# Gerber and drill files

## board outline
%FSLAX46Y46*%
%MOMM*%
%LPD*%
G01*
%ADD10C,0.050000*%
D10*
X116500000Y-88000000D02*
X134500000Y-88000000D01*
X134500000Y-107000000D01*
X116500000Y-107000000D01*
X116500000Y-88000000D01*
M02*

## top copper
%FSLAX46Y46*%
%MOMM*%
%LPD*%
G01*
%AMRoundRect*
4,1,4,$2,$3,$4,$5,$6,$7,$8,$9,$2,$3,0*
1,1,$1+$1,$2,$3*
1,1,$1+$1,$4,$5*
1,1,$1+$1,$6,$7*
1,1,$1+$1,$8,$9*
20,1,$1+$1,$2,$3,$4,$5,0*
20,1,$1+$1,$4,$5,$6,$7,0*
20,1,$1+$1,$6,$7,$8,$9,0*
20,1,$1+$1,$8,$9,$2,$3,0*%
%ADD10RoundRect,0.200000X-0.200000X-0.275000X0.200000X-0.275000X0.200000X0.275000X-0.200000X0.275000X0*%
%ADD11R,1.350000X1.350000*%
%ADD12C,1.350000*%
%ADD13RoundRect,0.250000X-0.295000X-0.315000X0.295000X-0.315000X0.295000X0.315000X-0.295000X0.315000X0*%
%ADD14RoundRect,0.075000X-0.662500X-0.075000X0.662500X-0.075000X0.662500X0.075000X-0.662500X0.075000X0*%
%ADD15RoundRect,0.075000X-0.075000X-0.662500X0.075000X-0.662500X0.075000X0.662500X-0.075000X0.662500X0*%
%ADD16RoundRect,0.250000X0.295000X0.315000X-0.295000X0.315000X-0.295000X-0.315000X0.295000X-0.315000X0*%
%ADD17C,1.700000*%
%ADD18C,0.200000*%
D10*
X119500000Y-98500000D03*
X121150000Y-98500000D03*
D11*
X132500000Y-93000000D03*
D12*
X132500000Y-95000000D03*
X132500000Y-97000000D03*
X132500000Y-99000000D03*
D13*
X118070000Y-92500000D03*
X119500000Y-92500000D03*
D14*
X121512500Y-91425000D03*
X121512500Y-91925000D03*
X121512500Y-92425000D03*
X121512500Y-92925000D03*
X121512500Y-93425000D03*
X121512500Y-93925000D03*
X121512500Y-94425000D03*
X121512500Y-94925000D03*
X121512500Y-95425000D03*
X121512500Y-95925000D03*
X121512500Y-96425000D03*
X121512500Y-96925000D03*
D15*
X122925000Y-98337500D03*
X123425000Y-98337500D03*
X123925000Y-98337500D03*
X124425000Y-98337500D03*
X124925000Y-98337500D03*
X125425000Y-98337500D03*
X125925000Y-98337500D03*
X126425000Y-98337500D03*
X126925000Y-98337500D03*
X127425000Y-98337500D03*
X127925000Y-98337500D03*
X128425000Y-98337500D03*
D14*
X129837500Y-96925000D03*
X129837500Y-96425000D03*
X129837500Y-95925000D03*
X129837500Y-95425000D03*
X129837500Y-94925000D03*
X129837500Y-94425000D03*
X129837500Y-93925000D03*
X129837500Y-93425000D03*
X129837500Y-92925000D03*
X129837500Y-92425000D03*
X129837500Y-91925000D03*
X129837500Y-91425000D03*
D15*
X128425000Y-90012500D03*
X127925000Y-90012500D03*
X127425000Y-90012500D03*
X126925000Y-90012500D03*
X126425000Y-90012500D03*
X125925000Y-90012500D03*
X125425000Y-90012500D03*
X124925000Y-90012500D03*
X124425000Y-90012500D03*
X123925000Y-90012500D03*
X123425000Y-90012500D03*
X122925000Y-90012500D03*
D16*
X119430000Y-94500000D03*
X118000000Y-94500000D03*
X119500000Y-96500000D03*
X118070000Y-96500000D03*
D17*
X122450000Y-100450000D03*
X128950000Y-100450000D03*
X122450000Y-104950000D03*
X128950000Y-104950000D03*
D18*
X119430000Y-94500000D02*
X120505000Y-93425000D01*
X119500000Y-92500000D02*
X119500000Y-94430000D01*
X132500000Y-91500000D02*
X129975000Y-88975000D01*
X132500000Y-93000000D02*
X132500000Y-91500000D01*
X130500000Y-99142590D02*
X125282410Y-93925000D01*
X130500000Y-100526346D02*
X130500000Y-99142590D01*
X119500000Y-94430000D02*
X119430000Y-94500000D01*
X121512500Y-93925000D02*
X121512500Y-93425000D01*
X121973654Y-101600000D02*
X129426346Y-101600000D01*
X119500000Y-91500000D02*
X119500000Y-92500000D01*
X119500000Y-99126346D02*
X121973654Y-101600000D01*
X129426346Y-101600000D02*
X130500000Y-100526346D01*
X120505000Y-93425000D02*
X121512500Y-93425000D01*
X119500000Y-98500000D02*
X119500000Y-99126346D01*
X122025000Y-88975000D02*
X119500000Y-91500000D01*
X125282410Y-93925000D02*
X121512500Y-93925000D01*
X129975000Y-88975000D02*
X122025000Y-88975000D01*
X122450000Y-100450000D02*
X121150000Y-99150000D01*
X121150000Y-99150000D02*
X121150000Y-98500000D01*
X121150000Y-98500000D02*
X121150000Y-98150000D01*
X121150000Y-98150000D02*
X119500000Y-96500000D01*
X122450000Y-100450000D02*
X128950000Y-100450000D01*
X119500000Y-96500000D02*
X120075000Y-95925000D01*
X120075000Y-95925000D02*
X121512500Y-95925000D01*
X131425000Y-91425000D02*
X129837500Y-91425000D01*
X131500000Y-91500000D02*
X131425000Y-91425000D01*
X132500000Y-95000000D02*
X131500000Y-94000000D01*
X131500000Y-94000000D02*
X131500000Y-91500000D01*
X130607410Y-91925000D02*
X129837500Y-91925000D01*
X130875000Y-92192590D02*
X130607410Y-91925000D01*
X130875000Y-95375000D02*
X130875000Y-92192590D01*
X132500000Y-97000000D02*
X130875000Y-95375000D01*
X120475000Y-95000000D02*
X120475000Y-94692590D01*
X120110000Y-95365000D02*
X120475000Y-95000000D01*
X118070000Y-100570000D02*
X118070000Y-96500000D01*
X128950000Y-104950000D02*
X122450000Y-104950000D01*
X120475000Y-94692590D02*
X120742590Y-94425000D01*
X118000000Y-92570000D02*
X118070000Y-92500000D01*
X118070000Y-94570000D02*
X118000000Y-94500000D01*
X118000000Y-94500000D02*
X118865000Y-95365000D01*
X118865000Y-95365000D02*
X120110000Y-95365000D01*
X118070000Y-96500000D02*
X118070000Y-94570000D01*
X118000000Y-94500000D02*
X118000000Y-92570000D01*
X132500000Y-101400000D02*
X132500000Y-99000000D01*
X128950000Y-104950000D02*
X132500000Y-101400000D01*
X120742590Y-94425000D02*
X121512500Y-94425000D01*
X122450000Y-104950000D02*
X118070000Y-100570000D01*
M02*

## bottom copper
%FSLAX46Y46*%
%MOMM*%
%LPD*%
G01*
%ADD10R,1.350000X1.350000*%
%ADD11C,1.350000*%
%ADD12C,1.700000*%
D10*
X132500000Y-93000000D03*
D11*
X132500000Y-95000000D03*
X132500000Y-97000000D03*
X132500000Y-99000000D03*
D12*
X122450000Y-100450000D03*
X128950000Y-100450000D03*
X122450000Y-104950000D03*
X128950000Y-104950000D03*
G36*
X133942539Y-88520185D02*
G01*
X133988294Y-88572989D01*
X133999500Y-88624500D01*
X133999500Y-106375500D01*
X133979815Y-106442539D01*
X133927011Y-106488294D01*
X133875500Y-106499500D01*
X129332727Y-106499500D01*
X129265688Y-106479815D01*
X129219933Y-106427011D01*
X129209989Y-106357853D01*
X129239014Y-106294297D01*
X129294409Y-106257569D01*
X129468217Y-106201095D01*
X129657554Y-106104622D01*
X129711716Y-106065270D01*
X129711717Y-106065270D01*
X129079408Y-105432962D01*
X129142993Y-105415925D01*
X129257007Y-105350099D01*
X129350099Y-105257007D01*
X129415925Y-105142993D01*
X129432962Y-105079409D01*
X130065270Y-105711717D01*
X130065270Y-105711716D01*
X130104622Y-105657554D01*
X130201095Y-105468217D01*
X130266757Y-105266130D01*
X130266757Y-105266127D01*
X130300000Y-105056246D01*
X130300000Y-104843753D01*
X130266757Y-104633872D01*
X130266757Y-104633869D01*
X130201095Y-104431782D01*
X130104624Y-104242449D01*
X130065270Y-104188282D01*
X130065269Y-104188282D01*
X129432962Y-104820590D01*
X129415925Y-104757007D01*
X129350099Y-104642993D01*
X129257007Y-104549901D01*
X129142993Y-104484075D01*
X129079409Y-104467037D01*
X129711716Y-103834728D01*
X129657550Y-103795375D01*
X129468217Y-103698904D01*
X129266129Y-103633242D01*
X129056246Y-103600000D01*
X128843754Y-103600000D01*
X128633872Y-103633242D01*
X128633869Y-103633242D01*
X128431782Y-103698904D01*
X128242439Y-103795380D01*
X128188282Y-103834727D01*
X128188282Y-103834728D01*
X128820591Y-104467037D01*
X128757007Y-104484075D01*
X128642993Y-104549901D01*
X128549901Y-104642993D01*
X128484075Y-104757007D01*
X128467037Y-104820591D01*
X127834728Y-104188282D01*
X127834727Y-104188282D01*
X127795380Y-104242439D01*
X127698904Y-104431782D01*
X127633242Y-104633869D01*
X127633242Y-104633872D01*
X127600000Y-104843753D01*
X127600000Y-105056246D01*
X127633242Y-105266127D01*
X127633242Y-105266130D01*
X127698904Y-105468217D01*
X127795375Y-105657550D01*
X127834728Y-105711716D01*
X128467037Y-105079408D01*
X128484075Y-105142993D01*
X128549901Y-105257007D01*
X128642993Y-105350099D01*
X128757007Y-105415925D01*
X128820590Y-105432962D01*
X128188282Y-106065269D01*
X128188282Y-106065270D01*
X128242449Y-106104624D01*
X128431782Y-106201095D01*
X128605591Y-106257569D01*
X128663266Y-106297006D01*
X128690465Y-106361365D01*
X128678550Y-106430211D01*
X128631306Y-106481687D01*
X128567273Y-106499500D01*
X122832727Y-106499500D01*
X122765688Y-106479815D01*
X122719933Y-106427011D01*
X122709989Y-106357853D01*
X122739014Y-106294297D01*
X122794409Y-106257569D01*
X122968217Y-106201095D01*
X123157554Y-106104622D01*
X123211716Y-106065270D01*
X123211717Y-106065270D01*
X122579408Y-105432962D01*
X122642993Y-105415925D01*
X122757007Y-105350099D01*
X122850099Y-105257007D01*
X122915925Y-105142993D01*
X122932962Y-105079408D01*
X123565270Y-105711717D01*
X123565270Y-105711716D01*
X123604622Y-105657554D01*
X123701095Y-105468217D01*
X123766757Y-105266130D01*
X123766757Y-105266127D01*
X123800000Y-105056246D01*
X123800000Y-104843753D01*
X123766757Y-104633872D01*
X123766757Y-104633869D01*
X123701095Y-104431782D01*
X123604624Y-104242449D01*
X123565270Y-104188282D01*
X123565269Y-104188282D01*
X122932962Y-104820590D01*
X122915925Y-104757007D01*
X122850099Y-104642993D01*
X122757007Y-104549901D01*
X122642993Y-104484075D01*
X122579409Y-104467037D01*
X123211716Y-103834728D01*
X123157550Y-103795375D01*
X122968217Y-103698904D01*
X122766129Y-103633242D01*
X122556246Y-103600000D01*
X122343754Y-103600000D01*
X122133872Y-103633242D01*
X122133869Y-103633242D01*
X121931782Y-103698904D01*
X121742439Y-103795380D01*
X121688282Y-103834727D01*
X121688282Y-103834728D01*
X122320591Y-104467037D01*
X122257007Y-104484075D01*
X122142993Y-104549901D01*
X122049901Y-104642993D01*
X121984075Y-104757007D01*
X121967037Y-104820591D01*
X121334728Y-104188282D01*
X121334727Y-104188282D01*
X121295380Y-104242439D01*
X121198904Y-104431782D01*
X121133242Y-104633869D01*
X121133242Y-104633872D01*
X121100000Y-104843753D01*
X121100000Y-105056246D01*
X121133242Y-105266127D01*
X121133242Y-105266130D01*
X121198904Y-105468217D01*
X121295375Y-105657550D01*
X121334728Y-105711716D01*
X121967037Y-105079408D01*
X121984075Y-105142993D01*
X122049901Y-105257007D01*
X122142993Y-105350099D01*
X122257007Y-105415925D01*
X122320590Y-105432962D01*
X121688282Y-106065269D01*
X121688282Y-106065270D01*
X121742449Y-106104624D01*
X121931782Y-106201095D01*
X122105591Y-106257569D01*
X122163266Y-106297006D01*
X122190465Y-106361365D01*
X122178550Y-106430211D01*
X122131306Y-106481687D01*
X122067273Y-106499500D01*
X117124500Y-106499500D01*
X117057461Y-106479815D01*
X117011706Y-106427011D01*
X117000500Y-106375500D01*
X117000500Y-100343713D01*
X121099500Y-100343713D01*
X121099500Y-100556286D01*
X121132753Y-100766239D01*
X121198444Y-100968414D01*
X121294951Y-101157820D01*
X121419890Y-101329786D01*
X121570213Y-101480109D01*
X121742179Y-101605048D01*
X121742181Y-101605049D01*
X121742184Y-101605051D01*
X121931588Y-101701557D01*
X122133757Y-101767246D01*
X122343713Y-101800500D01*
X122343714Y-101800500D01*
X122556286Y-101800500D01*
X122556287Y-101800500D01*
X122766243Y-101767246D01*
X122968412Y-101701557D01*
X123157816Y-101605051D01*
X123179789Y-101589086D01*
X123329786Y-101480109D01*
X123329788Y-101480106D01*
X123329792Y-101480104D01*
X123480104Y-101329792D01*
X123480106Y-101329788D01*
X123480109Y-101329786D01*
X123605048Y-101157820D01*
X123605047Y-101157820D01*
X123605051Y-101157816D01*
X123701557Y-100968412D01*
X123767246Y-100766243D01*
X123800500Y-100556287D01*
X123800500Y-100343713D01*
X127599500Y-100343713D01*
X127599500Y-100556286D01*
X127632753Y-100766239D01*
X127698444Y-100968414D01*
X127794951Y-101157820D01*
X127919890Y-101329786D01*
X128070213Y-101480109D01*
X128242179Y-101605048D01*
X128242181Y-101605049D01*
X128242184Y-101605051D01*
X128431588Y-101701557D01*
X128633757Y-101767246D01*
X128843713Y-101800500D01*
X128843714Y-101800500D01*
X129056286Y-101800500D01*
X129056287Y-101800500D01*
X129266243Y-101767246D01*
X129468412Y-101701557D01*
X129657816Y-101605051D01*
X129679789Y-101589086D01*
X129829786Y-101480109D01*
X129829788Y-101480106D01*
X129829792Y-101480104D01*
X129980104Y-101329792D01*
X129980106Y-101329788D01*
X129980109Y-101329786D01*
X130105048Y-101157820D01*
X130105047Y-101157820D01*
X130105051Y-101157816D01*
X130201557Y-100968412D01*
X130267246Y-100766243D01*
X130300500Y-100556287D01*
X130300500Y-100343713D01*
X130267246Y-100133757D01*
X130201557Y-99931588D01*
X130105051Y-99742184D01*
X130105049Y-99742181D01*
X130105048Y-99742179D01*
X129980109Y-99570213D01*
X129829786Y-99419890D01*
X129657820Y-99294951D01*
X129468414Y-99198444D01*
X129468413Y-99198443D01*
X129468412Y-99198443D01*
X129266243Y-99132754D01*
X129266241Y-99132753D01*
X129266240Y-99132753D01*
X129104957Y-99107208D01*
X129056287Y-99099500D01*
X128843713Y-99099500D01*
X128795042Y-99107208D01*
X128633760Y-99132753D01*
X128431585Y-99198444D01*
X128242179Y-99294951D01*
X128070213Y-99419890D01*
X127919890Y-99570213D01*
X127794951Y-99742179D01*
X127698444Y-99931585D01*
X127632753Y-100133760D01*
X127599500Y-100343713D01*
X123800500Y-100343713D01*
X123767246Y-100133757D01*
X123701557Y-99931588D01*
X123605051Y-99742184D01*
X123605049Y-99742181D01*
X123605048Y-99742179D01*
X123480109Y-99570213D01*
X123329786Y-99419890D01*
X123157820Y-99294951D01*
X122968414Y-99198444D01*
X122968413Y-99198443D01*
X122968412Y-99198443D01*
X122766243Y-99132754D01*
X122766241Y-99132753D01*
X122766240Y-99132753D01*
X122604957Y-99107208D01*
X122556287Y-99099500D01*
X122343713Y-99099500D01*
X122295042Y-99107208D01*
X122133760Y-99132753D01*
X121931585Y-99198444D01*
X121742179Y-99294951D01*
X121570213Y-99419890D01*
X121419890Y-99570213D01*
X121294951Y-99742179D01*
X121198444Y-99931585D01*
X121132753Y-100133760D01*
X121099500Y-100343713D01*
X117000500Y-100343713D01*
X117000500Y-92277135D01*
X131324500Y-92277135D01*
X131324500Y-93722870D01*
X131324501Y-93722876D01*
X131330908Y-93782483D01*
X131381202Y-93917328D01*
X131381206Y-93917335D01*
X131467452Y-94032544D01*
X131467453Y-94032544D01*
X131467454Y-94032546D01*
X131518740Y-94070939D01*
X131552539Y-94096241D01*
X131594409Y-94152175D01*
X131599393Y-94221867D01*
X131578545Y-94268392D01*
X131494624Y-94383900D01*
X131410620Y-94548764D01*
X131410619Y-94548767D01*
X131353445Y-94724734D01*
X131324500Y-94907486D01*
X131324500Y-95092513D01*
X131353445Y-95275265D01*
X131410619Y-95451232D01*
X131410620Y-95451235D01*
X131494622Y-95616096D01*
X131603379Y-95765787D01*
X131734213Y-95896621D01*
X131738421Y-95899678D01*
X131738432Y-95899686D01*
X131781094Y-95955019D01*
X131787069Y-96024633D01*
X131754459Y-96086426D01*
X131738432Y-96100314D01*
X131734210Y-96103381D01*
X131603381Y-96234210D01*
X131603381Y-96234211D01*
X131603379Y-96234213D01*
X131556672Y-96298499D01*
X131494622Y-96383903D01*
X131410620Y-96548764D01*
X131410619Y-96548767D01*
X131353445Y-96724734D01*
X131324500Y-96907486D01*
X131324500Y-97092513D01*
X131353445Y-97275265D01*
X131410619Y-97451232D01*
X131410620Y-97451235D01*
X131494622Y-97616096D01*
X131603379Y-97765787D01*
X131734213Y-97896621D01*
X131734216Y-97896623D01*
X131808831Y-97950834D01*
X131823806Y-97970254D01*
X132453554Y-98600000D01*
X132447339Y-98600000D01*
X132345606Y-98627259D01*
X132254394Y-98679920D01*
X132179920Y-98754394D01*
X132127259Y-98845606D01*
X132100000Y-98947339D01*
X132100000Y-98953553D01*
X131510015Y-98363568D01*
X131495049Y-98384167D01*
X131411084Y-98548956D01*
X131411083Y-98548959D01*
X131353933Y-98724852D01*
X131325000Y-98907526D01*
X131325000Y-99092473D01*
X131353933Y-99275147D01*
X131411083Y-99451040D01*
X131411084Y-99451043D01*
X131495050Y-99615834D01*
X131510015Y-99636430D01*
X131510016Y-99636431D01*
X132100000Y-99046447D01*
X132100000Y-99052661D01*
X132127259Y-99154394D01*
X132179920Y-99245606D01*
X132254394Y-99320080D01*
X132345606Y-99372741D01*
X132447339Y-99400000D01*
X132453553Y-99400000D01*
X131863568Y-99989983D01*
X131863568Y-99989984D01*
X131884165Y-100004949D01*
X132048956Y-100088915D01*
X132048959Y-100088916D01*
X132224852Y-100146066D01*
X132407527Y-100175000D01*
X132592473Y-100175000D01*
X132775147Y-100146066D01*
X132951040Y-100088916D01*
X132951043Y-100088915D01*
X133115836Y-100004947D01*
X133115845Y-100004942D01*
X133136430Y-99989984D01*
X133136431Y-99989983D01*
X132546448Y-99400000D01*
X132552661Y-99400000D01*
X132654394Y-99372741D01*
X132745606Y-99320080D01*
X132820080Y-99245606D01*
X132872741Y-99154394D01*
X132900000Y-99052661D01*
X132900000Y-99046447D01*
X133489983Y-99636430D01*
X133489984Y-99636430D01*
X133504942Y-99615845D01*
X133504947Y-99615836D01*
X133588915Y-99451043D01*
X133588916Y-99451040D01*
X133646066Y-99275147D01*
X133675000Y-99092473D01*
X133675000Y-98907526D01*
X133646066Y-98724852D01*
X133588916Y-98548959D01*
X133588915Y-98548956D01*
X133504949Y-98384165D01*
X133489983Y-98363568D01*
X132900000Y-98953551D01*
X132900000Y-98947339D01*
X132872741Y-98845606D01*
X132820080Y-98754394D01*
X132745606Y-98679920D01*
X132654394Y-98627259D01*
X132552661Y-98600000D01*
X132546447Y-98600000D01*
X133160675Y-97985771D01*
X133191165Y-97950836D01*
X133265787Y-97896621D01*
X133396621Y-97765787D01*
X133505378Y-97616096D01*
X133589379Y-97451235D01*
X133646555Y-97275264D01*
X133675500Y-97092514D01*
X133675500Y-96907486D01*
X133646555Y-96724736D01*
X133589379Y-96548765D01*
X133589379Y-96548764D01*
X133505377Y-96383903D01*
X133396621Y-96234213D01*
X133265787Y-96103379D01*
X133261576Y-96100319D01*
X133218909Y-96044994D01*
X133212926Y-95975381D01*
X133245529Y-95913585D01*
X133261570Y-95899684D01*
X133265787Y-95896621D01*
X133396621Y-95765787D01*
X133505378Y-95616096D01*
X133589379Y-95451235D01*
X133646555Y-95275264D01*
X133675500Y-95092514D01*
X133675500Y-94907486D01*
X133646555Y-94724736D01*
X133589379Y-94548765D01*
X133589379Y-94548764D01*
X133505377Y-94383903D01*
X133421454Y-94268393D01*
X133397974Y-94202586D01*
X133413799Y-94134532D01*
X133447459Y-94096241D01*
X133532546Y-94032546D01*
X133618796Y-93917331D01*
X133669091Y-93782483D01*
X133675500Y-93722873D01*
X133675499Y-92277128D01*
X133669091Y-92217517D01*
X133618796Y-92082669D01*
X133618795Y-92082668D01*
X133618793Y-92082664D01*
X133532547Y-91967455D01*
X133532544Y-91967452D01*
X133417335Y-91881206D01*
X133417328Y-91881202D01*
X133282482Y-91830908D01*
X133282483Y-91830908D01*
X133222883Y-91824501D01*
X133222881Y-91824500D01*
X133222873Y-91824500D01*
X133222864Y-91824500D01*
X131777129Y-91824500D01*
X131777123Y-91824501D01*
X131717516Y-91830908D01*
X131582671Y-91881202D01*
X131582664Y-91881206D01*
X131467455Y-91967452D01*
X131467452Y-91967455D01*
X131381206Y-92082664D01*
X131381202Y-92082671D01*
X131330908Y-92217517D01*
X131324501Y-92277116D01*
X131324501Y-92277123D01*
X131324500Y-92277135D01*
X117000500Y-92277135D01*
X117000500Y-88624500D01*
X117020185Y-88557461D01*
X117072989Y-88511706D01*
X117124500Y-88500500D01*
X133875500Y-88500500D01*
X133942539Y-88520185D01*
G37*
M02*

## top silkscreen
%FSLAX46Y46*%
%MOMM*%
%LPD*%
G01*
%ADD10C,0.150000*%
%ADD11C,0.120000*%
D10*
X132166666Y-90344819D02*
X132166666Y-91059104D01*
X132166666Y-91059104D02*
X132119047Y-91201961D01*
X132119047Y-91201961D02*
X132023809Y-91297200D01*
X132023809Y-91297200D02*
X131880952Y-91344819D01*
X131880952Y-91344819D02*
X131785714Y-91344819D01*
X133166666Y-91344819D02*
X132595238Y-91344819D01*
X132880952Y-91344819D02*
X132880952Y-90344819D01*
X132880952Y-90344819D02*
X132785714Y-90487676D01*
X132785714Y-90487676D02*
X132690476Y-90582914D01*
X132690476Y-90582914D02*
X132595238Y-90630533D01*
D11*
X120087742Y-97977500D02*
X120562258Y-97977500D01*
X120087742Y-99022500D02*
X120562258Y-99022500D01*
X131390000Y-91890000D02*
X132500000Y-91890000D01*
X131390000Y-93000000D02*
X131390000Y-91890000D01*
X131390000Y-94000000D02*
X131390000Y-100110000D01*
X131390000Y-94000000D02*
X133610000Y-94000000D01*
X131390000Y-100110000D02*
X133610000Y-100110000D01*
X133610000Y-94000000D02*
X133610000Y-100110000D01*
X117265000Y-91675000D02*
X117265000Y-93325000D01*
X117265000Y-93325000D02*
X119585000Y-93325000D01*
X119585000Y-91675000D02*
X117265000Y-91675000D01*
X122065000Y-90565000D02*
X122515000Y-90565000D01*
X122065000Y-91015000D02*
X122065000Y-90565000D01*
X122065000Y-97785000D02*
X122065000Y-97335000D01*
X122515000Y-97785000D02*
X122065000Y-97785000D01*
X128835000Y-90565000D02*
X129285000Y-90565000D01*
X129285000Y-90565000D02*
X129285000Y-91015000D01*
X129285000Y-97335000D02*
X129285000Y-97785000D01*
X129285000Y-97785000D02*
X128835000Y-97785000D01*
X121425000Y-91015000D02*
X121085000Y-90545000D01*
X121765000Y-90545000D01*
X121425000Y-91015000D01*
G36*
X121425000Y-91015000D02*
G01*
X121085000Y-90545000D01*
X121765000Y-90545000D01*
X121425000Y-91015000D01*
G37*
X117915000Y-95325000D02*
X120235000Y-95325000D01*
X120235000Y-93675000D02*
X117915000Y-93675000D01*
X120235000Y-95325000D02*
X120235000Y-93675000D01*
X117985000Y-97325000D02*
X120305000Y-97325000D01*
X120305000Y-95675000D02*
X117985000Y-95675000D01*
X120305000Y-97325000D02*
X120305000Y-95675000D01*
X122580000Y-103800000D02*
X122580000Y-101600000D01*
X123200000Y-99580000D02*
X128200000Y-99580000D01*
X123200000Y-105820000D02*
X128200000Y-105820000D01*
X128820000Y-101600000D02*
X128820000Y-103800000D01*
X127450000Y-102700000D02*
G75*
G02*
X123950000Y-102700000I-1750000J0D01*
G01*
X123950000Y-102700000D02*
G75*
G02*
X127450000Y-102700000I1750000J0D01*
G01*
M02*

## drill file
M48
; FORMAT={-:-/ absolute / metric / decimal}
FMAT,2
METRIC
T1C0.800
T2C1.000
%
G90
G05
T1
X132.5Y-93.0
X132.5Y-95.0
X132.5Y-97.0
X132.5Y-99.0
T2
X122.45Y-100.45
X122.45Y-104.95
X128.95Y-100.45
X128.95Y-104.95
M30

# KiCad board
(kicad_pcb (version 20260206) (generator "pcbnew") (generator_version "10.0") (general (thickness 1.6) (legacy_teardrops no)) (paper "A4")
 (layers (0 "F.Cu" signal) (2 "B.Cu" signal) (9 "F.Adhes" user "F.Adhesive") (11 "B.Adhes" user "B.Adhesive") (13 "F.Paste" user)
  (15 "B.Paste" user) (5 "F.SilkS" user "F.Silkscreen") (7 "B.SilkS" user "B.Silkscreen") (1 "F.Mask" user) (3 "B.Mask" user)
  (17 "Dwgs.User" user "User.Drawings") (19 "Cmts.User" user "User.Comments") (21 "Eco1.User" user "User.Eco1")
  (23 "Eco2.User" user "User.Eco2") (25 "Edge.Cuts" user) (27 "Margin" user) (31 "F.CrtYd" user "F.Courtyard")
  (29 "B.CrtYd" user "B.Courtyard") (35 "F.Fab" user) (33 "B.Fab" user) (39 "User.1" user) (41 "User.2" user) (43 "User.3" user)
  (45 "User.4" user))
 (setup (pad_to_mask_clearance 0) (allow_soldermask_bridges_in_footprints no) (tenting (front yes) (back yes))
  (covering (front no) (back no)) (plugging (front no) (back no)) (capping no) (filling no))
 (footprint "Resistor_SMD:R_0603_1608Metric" (layer "F.Cu") (at 120.325 98.5)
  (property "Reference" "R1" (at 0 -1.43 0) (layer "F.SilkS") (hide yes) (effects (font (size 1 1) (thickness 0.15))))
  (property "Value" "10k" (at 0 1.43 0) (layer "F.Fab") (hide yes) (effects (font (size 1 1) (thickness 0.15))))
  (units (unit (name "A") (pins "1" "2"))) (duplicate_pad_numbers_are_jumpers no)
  (fp_line (start -0.237258 -0.5225) (end 0.237258 -0.5225) (stroke (width 0.12) (type solid)) (layer "F.SilkS"))
  (fp_line (start -0.237258 0.5225) (end 0.237258 0.5225) (stroke (width 0.12) (type solid)) (layer "F.SilkS"))
  (pad "1" smd roundrect (at -0.825 0) (size 0.8 0.95) (layers "F.Cu" "F.Mask" "F.Paste") (roundrect_rratio 0.25) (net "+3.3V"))
  (pad "2" smd roundrect (at 0.825 0) (size 0.8 0.95) (layers "F.Cu" "F.Mask" "F.Paste") (roundrect_rratio 0.25) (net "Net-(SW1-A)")))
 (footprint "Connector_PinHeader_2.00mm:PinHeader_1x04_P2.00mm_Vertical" (layer "F.Cu") (at 132.5 93)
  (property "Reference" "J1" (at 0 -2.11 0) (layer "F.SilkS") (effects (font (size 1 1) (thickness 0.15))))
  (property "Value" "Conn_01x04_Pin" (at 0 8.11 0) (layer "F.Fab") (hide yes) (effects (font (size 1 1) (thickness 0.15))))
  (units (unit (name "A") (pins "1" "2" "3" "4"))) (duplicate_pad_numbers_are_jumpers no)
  (fp_line (start -1.11 -1.11) (end 0 -1.11) (stroke (width 0.12) (type solid)) (layer "F.SilkS"))
  (fp_line (start -1.11 0) (end -1.11 -1.11) (stroke (width 0.12) (type solid)) (layer "F.SilkS"))
  (fp_line (start -1.11 1) (end -1.11 7.11) (stroke (width 0.12) (type solid)) (layer "F.SilkS"))
  (fp_line (start -1.11 1) (end 1.11 1) (stroke (width 0.12) (type solid)) (layer "F.SilkS"))
  (fp_line (start -1.11 7.11) (end 1.11 7.11) (stroke (width 0.12) (type solid)) (layer "F.SilkS"))
  (fp_line (start 1.11 1) (end 1.11 7.11) (stroke (width 0.12) (type solid)) (layer "F.SilkS"))
  (pad "1" thru_hole rect (at 0 0) (size 1.35 1.35) (drill 0.8) (layers "*.Cu" "*.Mask") (remove_unused_layers no) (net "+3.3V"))
  (pad "2" thru_hole circle (at 0 2) (size 1.35 1.35) (drill 0.8) (layers "*.Cu" "*.Mask") (remove_unused_layers no) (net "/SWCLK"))
  (pad "3" thru_hole circle (at 0 4) (size 1.35 1.35) (drill 0.8) (layers "*.Cu" "*.Mask") (remove_unused_layers no) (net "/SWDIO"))
  (pad "4" thru_hole circle (at 0 6) (size 1.35 1.35) (drill 0.8) (layers "*.Cu" "*.Mask") (remove_unused_layers no) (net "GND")))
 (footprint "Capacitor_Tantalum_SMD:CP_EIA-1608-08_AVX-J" (layer "F.Cu") (at 118.785 92.5)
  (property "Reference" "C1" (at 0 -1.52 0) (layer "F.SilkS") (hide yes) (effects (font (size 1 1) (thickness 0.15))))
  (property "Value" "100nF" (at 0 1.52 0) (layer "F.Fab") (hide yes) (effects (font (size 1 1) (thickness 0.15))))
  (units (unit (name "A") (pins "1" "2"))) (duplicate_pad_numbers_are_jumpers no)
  (fp_line (start -1.52 -0.825) (end -1.52 0.825) (stroke (width 0.12) (type solid)) (layer "F.SilkS"))
  (fp_line (start -1.52 0.825) (end 0.8 0.825) (stroke (width 0.12) (type solid)) (layer "F.SilkS"))
  (fp_line (start 0.8 -0.825) (end -1.52 -0.825) (stroke (width 0.12) (type solid)) (layer "F.SilkS"))
  (pad "1" smd roundrect (at -0.715 0) (size 1.09 1.13) (layers "F.Cu" "F.Mask" "F.Paste") (roundrect_rratio 0.229358) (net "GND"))
  (pad "2" smd roundrect (at 0.715 0) (size 1.09 1.13) (layers "F.Cu" "F.Mask" "F.Paste") (roundrect_rratio 0.229358) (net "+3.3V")))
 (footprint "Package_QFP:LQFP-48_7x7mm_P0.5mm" (layer "F.Cu") (at 125.675 94.175)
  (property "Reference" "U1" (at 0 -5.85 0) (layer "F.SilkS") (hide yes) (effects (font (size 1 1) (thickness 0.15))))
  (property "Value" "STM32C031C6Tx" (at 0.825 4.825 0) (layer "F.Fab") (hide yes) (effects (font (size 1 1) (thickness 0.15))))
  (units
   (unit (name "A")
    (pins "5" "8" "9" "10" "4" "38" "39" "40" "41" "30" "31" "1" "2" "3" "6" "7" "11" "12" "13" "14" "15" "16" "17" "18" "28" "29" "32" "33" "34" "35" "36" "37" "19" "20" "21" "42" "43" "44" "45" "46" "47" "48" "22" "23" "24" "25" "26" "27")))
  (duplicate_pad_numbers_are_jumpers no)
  (fp_line (start -3.61 -3.61) (end -3.16 -3.61) (stroke (width 0.12) (type solid)) (layer "F.SilkS"))
  (fp_line (start -3.61 -3.16) (end -3.61 -3.61) (stroke (width 0.12) (type solid)) (layer "F.SilkS"))
  (fp_line (start -3.61 3.61) (end -3.61 3.16) (stroke (width 0.12) (type solid)) (layer "F.SilkS"))
  (fp_line (start -3.16 3.61) (end -3.61 3.61) (stroke (width 0.12) (type solid)) (layer "F.SilkS"))
  (fp_line (start 3.16 -3.61) (end 3.61 -3.61) (stroke (width 0.12) (type solid)) (layer "F.SilkS"))
  (fp_line (start 3.61 -3.61) (end 3.61 -3.16) (stroke (width 0.12) (type solid)) (layer "F.SilkS"))
  (fp_line (start 3.61 3.16) (end 3.61 3.61) (stroke (width 0.12) (type solid)) (layer "F.SilkS"))
  (fp_line (start 3.61 3.61) (end 3.16 3.61) (stroke (width 0.12) (type solid)) (layer "F.SilkS"))
  (fp_poly (pts (xy -4.25 -3.16) (xy -4.59 -3.63) (xy -3.91 -3.63)) (stroke (width 0.12) (type solid)) (fill yes) (layer "F.SilkS"))
  (pad "1" smd roundrect (at -4.1625 -2.75) (size 1.475 0.3) (layers "F.Cu" "F.Mask" "F.Paste") (roundrect_rratio 0.25)
   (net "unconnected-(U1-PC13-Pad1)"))
  (pad "2" smd roundrect (at -4.1625 -2.25) (size 1.475 0.3) (layers "F.Cu" "F.Mask" "F.Paste") (roundrect_rratio 0.25)
   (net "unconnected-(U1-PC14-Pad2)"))
  (pad "3" smd roundrect (at -4.1625 -1.75) (size 1.475 0.3) (layers "F.Cu" "F.Mask" "F.Paste") (roundrect_rratio 0.25)
   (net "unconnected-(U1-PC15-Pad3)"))
  (pad "4" smd roundrect (at -4.1625 -1.25) (size 1.475 0.3) (layers "F.Cu" "F.Mask" "F.Paste") (roundrect_rratio 0.25)
   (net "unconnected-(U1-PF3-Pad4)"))
  (pad "5" smd roundrect (at -4.1625 -0.75) (size 1.475 0.3) (layers "F.Cu" "F.Mask" "F.Paste") (roundrect_rratio 0.25) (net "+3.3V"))
  (pad "6" smd roundrect (at -4.1625 -0.25) (size 1.475 0.3) (layers "F.Cu" "F.Mask" "F.Paste") (roundrect_rratio 0.25) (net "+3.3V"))
  (pad "7" smd roundrect (at -4.1625 0.25) (size 1.475 0.3) (layers "F.Cu" "F.Mask" "F.Paste") (roundrect_rratio 0.25) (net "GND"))
  (pad "8" smd roundrect (at -4.1625 0.75) (size 1.475 0.3) (layers "F.Cu" "F.Mask" "F.Paste") (roundrect_rratio 0.25)
   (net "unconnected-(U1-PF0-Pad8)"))
  (pad "9" smd roundrect (at -4.1625 1.25) (size 1.475 0.3) (layers "F.Cu" "F.Mask" "F.Paste") (roundrect_rratio 0.25)
   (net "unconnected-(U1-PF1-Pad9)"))
  (pad "10" smd roundrect (at -4.1625 1.75) (size 1.475 0.3) (layers "F.Cu" "F.Mask" "F.Paste") (roundrect_rratio 0.25) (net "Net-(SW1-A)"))
  (pad "11" smd roundrect (at -4.1625 2.25) (size 1.475 0.3) (layers "F.Cu" "F.Mask" "F.Paste") (roundrect_rratio 0.25)
   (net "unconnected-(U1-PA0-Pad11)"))
  (pad "12" smd roundrect (at -4.1625 2.75) (size 1.475 0.3) (layers "F.Cu" "F.Mask" "F.Paste") (roundrect_rratio 0.25)
   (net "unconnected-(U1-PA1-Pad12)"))
  (pad "13" smd roundrect (at -2.75 4.1625) (size 0.3 1.475) (layers "F.Cu" "F.Mask" "F.Paste") (roundrect_rratio 0.25)
   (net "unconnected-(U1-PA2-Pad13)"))
  (pad "14" smd roundrect (at -2.25 4.1625) (size 0.3 1.475) (layers "F.Cu" "F.Mask" "F.Paste") (roundrect_rratio 0.25)
   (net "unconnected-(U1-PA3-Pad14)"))
  (pad "15" smd roundrect (at -1.75 4.1625) (size 0.3 1.475) (layers "F.Cu" "F.Mask" "F.Paste") (roundrect_rratio 0.25)
   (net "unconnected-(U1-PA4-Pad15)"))
  (pad "16" smd roundrect (at -1.25 4.1625) (size 0.3 1.475) (layers "F.Cu" "F.Mask" "F.Paste") (roundrect_rratio 0.25)
   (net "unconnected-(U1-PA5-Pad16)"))
  (pad "17" smd roundrect (at -0.75 4.1625) (size 0.3 1.475) (layers "F.Cu" "F.Mask" "F.Paste") (roundrect_rratio 0.25)
   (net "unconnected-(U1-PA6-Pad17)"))
  (pad "18" smd roundrect (at -0.25 4.1625) (size 0.3 1.475) (layers "F.Cu" "F.Mask" "F.Paste") (roundrect_rratio 0.25)
   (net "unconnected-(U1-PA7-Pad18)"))
  (pad "19" smd roundrect (at 0.25 4.1625) (size 0.3 1.475) (layers "F.Cu" "F.Mask" "F.Paste") (roundrect_rratio 0.25)
   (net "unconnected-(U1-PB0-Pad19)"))
  (pad "20" smd roundrect (at 0.75 4.1625) (size 0.3 1.475) (layers "F.Cu" "F.Mask" "F.Paste") (roundrect_rratio 0.25)
   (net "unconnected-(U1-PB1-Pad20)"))
  (pad "21" smd roundrect (at 1.25 4.1625) (size 0.3 1.475) (layers "F.Cu" "F.Mask" "F.Paste") (roundrect_rratio 0.25)
   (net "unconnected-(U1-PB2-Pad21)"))
  (pad "22" smd roundrect (at 1.75 4.1625) (size 0.3 1.475) (layers "F.Cu" "F.Mask" "F.Paste") (roundrect_rratio 0.25)
   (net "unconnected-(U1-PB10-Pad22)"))
  (pad "23" smd roundrect (at 2.25 4.1625) (size 0.3 1.475) (layers "F.Cu" "F.Mask" "F.Paste") (roundrect_rratio 0.25)
   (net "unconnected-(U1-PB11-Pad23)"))
  (pad "24" smd roundrect (at 2.75 4.1625) (size 0.3 1.475) (layers "F.Cu" "F.Mask" "F.Paste") (roundrect_rratio 0.25)
   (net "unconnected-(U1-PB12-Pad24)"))
  (pad "25" smd roundrect (at 4.1625 2.75) (size 1.475 0.3) (layers "F.Cu" "F.Mask" "F.Paste") (roundrect_rratio 0.25)
   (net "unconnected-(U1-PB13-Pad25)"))
  (pad "26" smd roundrect (at 4.1625 2.25) (size 1.475 0.3) (layers "F.Cu" "F.Mask" "F.Paste") (roundrect_rratio 0.25)
   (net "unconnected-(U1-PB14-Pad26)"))
  (pad "27" smd roundrect (at 4.1625 1.75) (size 1.475 0.3) (layers "F.Cu" "F.Mask" "F.Paste") (roundrect_rratio 0.25)
   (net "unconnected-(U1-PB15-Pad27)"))
  (pad "28" smd roundrect (at 4.1625 1.25) (size 1.475 0.3) (layers "F.Cu" "F.Mask" "F.Paste") (roundrect_rratio 0.25)
   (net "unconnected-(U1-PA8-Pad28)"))
  (pad "29" smd roundrect (at 4.1625 0.75) (size 1.475 0.3) (layers "F.Cu" "F.Mask" "F.Paste") (roundrect_rratio 0.25)
   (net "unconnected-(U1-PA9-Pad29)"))
  (pad "30" smd roundrect (at 4.1625 0.25) (size 1.475 0.3) (layers "F.Cu" "F.Mask" "F.Paste") (roundrect_rratio 0.25)
   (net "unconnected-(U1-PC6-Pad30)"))
  (pad "31" smd roundrect (at 4.1625 -0.25) (size 1.475 0.3) (layers "F.Cu" "F.Mask" "F.Paste") (roundrect_rratio 0.25)
   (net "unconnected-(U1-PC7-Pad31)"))
  (pad "32" smd roundrect (at 4.1625 -0.75) (size 1.475 0.3) (layers "F.Cu" "F.Mask" "F.Paste") (roundrect_rratio 0.25)
   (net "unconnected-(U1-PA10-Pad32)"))
  (pad "33" smd roundrect (at 4.1625 -1.25) (size 1.475 0.3) (layers "F.Cu" "F.Mask" "F.Paste") (roundrect_rratio 0.25)
   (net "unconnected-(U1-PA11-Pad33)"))
  (pad "34" smd roundrect (at 4.1625 -1.75) (size 1.475 0.3) (layers "F.Cu" "F.Mask" "F.Paste") (roundrect_rratio 0.25)
   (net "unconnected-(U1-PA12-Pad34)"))
  (pad "35" smd roundrect (at 4.1625 -2.25) (size 1.475 0.3) (layers "F.Cu" "F.Mask" "F.Paste") (roundrect_rratio 0.25) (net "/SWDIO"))
  (pad "36" smd roundrect (at 4.1625 -2.75) (size 1.475 0.3) (layers "F.Cu" "F.Mask" "F.Paste") (roundrect_rratio 0.25) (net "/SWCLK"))
  (pad "37" smd roundrect (at 2.75 -4.1625) (size 0.3 1.475) (layers "F.Cu" "F.Mask" "F.Paste") (roundrect_rratio 0.25)
   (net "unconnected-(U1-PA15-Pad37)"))
  (pad "38" smd roundrect (at 2.25 -4.1625) (size 0.3 1.475) (layers "F.Cu" "F.Mask" "F.Paste") (roundrect_rratio 0.25)
   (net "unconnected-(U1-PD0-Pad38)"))
  (pad "39" smd roundrect (at 1.75 -4.1625) (size 0.3 1.475) (layers "F.Cu" "F.Mask" "F.Paste") (roundrect_rratio 0.25)
   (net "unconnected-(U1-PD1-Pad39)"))
  (pad "40" smd roundrect (at 1.25 -4.1625) (size 0.3 1.475) (layers "F.Cu" "F.Mask" "F.Paste") (roundrect_rratio 0.25)
   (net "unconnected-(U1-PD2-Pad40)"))
  (pad "41" smd roundrect (at 0.75 -4.1625) (size 0.3 1.475) (layers "F.Cu" "F.Mask" "F.Paste") (roundrect_rratio 0.25)
   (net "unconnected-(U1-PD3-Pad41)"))
  (pad "42" smd roundrect (at 0.25 -4.1625) (size 0.3 1.475) (layers "F.Cu" "F.Mask" "F.Paste") (roundrect_rratio 0.25)
   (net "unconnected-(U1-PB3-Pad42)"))
  (pad "43" smd roundrect (at -0.25 -4.1625) (size 0.3 1.475) (layers "F.Cu" "F.Mask" "F.Paste") (roundrect_rratio 0.25)
   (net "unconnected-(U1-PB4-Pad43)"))
  (pad "44" smd roundrect (at -0.75 -4.1625) (size 0.3 1.475) (layers "F.Cu" "F.Mask" "F.Paste") (roundrect_rratio 0.25)
   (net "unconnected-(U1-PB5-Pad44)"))
  (pad "45" smd roundrect (at -1.25 -4.1625) (size 0.3 1.475) (layers "F.Cu" "F.Mask" "F.Paste") (roundrect_rratio 0.25)
   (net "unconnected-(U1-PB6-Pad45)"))
  (pad "46" smd roundrect (at -1.75 -4.1625) (size 0.3 1.475) (layers "F.Cu" "F.Mask" "F.Paste") (roundrect_rratio 0.25)
   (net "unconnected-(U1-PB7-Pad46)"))
  (pad "47" smd roundrect (at -2.25 -4.1625) (size 0.3 1.475) (layers "F.Cu" "F.Mask" "F.Paste") (roundrect_rratio 0.25)
   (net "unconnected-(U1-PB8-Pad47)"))
  (pad "48" smd roundrect (at -2.75 -4.1625) (size 0.3 1.475) (layers "F.Cu" "F.Mask" "F.Paste") (roundrect_rratio 0.25)
   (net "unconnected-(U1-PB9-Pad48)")))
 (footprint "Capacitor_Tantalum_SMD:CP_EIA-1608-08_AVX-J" (layer "F.Cu") (at 118.715 94.5 180)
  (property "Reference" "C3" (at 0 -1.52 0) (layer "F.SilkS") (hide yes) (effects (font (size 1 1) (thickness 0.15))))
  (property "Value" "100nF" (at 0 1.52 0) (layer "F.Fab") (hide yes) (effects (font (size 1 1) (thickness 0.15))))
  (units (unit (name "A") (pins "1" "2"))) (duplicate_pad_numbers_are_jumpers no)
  (fp_line (start 0.8 -0.825) (end -1.52 -0.825) (stroke (width 0.12) (type solid)) (layer "F.SilkS"))
  (fp_line (start -1.52 0.825) (end 0.8 0.825) (stroke (width 0.12) (type solid)) (layer "F.SilkS"))
  (fp_line (start -1.52 -0.825) (end -1.52 0.825) (stroke (width 0.12) (type solid)) (layer "F.SilkS"))
  (pad "1" smd roundrect (at -0.715 0 180) (size 1.09 1.13) (layers "F.Cu" "F.Mask" "F.Paste") (roundrect_rratio 0.229358) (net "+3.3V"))
  (pad "2" smd roundrect (at 0.715 0 180) (size 1.09 1.13) (layers "F.Cu" "F.Mask" "F.Paste") (roundrect_rratio 0.229358) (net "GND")))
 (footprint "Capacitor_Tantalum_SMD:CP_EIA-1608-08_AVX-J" (layer "F.Cu") (at 118.785 96.5 180)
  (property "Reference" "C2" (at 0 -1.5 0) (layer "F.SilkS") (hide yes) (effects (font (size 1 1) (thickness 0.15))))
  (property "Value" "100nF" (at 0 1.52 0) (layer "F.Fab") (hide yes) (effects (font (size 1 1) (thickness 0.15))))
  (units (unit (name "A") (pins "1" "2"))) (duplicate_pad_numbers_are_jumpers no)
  (fp_line (start 0.8 -0.825) (end -1.52 -0.825) (stroke (width 0.12) (type solid)) (layer "F.SilkS"))
  (fp_line (start -1.52 0.825) (end 0.8 0.825) (stroke (width 0.12) (type solid)) (layer "F.SilkS"))
  (fp_line (start -1.52 -0.825) (end -1.52 0.825) (stroke (width 0.12) (type solid)) (layer "F.SilkS"))
  (pad "1" smd roundrect (at -0.715 0 180) (size 1.09 1.13) (layers "F.Cu" "F.Mask" "F.Paste") (roundrect_rratio 0.229358)
   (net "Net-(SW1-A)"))
  (pad "2" smd roundrect (at 0.715 0 180) (size 1.09 1.13) (layers "F.Cu" "F.Mask" "F.Paste") (roundrect_rratio 0.229358) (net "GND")))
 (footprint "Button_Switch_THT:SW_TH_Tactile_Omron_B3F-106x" (layer "F.Cu") (at 122.45 100.45)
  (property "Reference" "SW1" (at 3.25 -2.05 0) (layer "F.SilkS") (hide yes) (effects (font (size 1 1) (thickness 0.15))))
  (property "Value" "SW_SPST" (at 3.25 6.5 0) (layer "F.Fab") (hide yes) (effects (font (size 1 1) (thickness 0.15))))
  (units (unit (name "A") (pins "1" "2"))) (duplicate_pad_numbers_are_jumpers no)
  (fp_line (start 0.13 3.35) (end 0.13 1.15) (stroke (width 0.12) (type solid)) (layer "F.SilkS"))
  (fp_line (start 0.75 -0.87) (end 5.75 -0.87) (stroke (width 0.12) (type solid)) (layer "F.SilkS"))
  (fp_line (start 0.75 5.37) (end 5.75 5.37) (stroke (width 0.12) (type solid)) (layer "F.SilkS"))
  (fp_line (start 6.37 1.15) (end 6.37 3.35) (stroke (width 0.12) (type solid)) (layer "F.SilkS"))
  (fp_circle (center 3.25 2.25) (end 5 2.25) (stroke (width 0.12) (type solid)) (fill no) (layer "F.SilkS"))
  (pad "1" thru_hole circle (at 0 0) (size 1.7 1.7) (drill 1) (layers "*.Cu" "*.Mask") (remove_unused_layers no) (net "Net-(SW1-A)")
   (thermal_bridge_angle 90))
  (pad "1" thru_hole circle (at 6.5 0) (size 1.7 1.7) (drill 1) (layers "*.Cu" "*.Mask") (remove_unused_layers no) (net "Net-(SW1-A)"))
  (pad "2" thru_hole circle (at 0 4.5) (size 1.7 1.7) (drill 1) (layers "*.Cu" "*.Mask") (remove_unused_layers no) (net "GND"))
  (pad "2" thru_hole circle (at 6.5 4.5) (size 1.7 1.7) (drill 1) (layers "*.Cu" "*.Mask") (remove_unused_layers no) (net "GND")))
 (gr_rect (start 116.5 88) (end 134.5 107) (stroke (width 0.05) (type default)) (fill no) (layer "Edge.Cuts"))
 (segment (start 119.43 94.5) (end 120.505 93.425) (width 0.2) (layer "F.Cu") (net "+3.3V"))
 (segment (start 119.5 92.5) (end 119.5 94.43) (width 0.2) (layer "F.Cu") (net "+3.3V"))
 (segment (start 132.5 91.5) (end 129.975 88.975) (width 0.2) (layer "F.Cu") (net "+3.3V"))
 (segment (start 132.5 93) (end 132.5 91.5) (width 0.2) (layer "F.Cu") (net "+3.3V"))
 (segment (start 130.5 99.14259) (end 125.28241 93.925) (width 0.2) (layer "F.Cu") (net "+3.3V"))
 (segment (start 130.5 100.526346) (end 130.5 99.14259) (width 0.2) (layer "F.Cu") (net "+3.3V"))
 (segment (start 119.5 94.43) (end 119.43 94.5) (width 0.2) (layer "F.Cu") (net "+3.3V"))
 (segment (start 121.5125 93.925) (end 121.5125 93.425) (width 0.2) (layer "F.Cu") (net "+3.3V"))
 (segment (start 121.973654 101.6) (end 129.426346 101.6) (width 0.2) (layer "F.Cu") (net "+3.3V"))
 (segment (start 119.5 91.5) (end 119.5 92.5) (width 0.2) (layer "F.Cu") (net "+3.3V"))
 (segment (start 119.5 99.126346) (end 121.973654 101.6) (width 0.2) (layer "F.Cu") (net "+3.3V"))
 (segment (start 129.426346 101.6) (end 130.5 100.526346) (width 0.2) (layer "F.Cu") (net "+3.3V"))
 (segment (start 120.505 93.425) (end 121.5125 93.425) (width 0.2) (layer "F.Cu") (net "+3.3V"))
 (segment (start 119.5 98.5) (end 119.5 99.126346) (width 0.2) (layer "F.Cu") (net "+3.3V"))
 (segment (start 122.025 88.975) (end 119.5 91.5) (width 0.2) (layer "F.Cu") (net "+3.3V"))
 (segment (start 125.28241 93.925) (end 121.5125 93.925) (width 0.2) (layer "F.Cu") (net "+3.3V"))
 (segment (start 129.975 88.975) (end 122.025 88.975) (width 0.2) (layer "F.Cu") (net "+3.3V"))
 (segment (start 122.45 100.45) (end 121.15 99.15) (width 0.2) (layer "F.Cu") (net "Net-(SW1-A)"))
 (segment (start 121.15 99.15) (end 121.15 98.5) (width 0.2) (layer "F.Cu") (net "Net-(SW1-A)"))
 (segment (start 121.15 98.5) (end 121.15 98.15) (width 0.2) (layer "F.Cu") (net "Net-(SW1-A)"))
 (segment (start 121.15 98.15) (end 119.5 96.5) (width 0.2) (layer "F.Cu") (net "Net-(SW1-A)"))
 (segment (start 122.45 100.45) (end 128.95 100.45) (width 0.2) (layer "F.Cu") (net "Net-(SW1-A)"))
 (segment (start 119.5 96.5) (end 120.075 95.925) (width 0.2) (layer "F.Cu") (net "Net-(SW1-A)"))
 (segment (start 120.075 95.925) (end 121.5125 95.925) (width 0.2) (layer "F.Cu") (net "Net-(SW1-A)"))
 (segment (start 131.425 91.425) (end 129.8375 91.425) (width 0.2) (layer "F.Cu") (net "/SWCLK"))
 (segment (start 131.5 91.5) (end 131.425 91.425) (width 0.2) (layer "F.Cu") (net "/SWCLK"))
 (segment (start 132.5 95) (end 131.5 94) (width 0.2) (layer "F.Cu") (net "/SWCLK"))
 (segment (start 131.5 94) (end 131.5 91.5) (width 0.2) (layer "F.Cu") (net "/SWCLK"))
 (segment (start 130.60741 91.925) (end 129.8375 91.925) (width 0.2) (layer "F.Cu") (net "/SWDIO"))
 (segment (start 130.875 92.19259) (end 130.60741 91.925) (width 0.2) (layer "F.Cu") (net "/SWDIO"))
 (segment (start 130.875 95.375) (end 130.875 92.19259) (width 0.2) (layer "F.Cu") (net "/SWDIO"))
 (segment (start 132.5 97) (end 130.875 95.375) (width 0.2) (layer "F.Cu") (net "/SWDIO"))
 (segment (start 120.475 95) (end 120.475 94.69259) (width 0.2) (layer "F.Cu") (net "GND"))
 (segment (start 120.11 95.365) (end 120.475 95) (width 0.2) (layer "F.Cu") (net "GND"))
 (segment (start 118.07 100.57) (end 118.07 96.5) (width 0.2) (layer "F.Cu") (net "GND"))
 (segment (start 128.95 104.95) (end 122.45 104.95) (width 0.2) (layer "F.Cu") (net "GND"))
 (segment (start 120.475 94.69259) (end 120.74259 94.425) (width 0.2) (layer "F.Cu") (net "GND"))
 (segment (start 118 92.57) (end 118.07 92.5) (width 0.2) (layer "F.Cu") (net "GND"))
 (segment (start 118.07 94.57) (end 118 94.5) (width 0.2) (layer "F.Cu") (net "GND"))
 (segment (start 118 94.5) (end 118.865 95.365) (width 0.2) (layer "F.Cu") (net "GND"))
 (segment (start 118.865 95.365) (end 120.11 95.365) (width 0.2) (layer "F.Cu") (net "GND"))
 (segment (start 118.07 96.5) (end 118.07 94.57) (width 0.2) (layer "F.Cu") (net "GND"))
 (segment (start 118 94.5) (end 118 92.57) (width 0.2) (layer "F.Cu") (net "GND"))
 (segment (start 132.5 101.4) (end 132.5 99) (width 0.2) (layer "F.Cu") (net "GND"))
 (segment (start 128.95 104.95) (end 132.5 101.4) (width 0.2) (layer "F.Cu") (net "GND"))
 (segment (start 120.74259 94.425) (end 121.5125 94.425) (width 0.2) (layer "F.Cu") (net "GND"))
 (segment (start 122.45 104.95) (end 118.07 100.57) (width 0.2) (layer "F.Cu") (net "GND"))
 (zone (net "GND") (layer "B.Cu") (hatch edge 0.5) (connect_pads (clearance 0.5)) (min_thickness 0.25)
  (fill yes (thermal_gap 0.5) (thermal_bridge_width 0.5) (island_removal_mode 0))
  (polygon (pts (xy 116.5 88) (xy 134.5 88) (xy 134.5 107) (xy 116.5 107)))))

